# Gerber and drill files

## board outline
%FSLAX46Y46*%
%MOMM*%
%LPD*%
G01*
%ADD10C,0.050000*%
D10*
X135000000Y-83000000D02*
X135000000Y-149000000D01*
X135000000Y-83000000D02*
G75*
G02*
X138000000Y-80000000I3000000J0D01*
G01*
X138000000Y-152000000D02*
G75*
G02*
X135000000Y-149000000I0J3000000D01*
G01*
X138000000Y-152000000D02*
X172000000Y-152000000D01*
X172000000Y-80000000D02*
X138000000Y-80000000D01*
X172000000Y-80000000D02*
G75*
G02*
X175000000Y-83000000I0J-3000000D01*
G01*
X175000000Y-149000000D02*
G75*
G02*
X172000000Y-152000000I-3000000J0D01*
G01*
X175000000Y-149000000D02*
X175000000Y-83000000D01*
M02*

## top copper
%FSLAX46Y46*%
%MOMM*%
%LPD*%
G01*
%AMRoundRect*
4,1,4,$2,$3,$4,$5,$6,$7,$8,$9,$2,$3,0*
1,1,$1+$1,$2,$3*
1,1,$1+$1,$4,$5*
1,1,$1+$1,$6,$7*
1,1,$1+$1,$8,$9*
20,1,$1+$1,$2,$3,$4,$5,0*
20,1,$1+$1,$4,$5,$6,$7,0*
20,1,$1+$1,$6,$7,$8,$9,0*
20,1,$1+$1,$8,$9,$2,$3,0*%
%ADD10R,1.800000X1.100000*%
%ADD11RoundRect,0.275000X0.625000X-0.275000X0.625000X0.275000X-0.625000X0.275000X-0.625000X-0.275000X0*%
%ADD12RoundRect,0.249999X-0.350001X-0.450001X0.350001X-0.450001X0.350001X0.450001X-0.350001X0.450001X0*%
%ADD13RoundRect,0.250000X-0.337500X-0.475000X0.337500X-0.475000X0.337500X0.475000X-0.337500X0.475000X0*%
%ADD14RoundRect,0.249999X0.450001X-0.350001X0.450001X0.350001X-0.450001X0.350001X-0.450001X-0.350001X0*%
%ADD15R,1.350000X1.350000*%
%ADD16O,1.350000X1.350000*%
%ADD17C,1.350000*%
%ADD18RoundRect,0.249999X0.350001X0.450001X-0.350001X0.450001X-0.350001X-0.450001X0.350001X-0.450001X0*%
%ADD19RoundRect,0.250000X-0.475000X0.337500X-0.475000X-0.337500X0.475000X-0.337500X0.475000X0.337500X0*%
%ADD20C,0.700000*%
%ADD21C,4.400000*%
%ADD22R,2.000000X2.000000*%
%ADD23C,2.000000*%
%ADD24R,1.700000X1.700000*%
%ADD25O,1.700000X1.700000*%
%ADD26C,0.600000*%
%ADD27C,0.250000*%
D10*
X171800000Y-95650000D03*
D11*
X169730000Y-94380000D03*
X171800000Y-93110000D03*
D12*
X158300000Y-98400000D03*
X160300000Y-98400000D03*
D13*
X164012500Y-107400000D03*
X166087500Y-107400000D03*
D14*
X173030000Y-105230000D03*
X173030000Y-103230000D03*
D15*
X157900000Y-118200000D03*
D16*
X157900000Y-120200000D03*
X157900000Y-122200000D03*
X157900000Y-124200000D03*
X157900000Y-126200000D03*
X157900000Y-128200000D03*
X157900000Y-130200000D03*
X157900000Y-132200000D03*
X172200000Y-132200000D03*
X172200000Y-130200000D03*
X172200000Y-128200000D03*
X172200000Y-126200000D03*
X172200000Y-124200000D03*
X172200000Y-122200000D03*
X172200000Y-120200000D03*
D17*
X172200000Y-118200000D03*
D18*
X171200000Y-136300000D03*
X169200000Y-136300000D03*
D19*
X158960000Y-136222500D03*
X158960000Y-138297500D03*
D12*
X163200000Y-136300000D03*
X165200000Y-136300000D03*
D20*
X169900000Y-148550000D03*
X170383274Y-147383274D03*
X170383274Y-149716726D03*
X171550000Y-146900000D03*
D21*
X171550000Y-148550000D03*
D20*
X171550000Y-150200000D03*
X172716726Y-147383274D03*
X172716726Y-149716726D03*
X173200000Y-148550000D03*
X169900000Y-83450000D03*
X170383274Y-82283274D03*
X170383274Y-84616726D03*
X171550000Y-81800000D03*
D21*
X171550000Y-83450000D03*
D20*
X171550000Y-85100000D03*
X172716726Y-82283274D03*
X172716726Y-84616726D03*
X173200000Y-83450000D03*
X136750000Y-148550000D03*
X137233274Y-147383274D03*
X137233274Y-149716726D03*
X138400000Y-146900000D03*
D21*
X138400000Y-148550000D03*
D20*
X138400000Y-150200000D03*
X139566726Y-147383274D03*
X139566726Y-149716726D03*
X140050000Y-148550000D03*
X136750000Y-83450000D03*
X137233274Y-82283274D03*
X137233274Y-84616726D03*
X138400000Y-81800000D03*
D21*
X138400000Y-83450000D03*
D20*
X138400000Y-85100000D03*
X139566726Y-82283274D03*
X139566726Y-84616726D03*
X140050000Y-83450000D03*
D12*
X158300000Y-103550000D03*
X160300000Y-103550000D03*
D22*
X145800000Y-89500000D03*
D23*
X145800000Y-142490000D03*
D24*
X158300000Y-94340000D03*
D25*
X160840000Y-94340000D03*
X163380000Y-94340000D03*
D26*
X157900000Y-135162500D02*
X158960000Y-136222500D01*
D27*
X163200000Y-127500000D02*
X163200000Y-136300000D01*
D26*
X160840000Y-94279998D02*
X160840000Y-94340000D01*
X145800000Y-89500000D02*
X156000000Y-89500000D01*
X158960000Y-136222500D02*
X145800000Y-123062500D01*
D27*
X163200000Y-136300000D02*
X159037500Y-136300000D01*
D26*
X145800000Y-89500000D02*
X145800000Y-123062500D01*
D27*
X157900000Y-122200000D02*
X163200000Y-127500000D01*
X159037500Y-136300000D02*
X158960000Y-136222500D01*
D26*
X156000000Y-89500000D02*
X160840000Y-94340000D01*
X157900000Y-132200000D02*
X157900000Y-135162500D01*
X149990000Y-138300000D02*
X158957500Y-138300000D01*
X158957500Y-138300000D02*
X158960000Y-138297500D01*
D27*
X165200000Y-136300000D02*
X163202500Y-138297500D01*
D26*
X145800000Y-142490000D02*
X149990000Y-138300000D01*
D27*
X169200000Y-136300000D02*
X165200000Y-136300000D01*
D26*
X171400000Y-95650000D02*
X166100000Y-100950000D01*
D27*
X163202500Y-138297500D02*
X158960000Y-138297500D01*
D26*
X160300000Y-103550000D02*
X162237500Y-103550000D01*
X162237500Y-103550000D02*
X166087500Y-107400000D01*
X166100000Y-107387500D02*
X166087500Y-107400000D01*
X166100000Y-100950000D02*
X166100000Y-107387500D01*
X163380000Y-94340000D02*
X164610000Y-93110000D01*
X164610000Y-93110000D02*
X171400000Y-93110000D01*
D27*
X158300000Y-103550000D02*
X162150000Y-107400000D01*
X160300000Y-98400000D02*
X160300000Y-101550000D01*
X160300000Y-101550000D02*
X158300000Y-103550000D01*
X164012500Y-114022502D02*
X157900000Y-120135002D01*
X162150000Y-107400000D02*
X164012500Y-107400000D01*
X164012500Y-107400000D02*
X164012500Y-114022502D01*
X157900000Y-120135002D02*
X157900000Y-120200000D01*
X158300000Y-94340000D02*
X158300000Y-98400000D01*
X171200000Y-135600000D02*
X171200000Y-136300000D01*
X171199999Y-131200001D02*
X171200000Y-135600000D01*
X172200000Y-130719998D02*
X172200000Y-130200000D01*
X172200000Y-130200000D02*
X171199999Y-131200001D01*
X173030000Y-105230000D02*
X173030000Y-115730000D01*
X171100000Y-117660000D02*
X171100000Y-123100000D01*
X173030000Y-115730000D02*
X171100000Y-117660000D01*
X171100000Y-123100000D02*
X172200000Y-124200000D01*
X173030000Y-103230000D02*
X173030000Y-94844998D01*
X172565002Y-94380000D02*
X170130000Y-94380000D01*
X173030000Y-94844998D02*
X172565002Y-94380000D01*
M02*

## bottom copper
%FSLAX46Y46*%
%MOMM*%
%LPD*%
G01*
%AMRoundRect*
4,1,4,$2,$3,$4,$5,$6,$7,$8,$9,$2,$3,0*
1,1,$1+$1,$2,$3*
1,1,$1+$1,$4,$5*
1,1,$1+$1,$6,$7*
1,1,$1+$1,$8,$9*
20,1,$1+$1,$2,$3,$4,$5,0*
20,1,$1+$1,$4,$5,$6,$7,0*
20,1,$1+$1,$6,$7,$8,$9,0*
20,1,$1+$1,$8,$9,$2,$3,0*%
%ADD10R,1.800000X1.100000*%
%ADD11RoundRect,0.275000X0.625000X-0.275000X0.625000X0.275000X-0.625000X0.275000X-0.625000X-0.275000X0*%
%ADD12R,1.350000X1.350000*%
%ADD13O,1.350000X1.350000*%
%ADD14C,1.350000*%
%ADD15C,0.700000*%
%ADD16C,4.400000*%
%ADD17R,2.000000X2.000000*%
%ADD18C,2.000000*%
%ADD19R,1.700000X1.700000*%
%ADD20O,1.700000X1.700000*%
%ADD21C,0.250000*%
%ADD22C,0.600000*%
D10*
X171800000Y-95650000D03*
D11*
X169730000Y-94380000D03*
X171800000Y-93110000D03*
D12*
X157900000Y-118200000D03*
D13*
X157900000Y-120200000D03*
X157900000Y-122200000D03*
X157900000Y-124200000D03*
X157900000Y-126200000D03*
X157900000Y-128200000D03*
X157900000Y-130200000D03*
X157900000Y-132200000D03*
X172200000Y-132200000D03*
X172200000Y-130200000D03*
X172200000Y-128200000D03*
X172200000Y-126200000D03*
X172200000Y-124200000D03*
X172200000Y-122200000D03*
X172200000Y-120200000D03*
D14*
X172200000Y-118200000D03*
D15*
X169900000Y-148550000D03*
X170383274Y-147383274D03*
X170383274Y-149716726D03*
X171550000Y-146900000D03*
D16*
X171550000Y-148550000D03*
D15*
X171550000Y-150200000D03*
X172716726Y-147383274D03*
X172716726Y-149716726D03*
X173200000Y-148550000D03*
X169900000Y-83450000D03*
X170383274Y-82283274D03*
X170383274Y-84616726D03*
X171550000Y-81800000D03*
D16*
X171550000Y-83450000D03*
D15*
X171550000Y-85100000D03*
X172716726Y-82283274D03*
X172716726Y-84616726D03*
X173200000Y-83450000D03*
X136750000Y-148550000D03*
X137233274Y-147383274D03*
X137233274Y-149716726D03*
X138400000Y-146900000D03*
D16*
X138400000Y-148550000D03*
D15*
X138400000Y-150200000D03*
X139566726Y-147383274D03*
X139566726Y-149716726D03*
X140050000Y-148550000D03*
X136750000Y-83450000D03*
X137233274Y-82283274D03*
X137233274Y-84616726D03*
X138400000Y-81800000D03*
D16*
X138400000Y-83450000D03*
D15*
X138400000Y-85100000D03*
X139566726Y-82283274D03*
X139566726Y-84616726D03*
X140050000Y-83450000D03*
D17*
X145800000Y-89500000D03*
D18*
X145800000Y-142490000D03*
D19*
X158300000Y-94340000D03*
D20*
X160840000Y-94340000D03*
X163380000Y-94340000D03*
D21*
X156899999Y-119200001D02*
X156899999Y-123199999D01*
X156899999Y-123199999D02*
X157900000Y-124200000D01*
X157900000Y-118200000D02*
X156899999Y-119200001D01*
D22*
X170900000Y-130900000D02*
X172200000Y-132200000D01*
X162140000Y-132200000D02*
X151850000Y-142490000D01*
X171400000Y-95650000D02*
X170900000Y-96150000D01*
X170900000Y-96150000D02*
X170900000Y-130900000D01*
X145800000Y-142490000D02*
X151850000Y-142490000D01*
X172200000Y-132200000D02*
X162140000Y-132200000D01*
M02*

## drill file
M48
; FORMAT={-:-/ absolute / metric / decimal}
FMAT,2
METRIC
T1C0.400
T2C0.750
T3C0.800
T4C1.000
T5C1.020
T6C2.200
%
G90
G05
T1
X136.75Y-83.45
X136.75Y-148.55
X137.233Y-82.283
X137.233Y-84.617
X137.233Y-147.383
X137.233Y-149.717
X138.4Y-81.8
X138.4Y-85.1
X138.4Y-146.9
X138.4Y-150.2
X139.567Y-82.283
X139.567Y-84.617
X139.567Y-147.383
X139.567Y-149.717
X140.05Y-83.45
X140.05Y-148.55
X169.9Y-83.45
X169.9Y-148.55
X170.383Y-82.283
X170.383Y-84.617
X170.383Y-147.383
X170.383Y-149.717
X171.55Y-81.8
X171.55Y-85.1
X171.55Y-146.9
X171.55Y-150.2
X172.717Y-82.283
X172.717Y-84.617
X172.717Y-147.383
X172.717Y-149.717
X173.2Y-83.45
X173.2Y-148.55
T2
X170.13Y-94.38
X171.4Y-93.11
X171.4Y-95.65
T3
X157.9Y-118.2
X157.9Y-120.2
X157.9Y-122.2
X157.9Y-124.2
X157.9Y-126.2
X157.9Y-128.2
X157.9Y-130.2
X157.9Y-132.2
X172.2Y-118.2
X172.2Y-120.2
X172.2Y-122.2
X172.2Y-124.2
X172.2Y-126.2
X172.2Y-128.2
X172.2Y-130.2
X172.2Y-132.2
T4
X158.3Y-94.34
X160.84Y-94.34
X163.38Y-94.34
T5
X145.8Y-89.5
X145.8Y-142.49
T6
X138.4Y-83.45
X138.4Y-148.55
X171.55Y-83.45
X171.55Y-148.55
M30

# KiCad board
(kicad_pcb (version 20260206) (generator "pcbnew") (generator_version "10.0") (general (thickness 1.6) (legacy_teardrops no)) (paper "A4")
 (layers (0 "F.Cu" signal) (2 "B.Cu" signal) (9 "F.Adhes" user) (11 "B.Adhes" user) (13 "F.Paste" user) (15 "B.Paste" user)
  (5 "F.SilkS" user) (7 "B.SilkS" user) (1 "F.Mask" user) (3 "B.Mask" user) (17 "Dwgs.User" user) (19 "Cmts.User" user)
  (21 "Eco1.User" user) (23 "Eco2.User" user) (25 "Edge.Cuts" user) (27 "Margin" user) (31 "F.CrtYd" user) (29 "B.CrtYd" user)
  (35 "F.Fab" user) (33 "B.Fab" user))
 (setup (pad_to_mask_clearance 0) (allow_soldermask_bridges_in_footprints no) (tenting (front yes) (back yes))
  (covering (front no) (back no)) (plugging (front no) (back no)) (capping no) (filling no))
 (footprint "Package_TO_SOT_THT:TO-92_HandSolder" (layer "F.Cu") (at 171.4 95.65 90)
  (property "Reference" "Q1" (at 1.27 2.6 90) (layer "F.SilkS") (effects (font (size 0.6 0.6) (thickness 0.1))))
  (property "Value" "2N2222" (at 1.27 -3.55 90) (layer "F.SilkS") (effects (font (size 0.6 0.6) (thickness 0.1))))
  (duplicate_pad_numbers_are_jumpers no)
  (pad "1" thru_hole rect (at 0 0 90) (size 1.1 1.8) (drill 0.75 (offset 0 0.4)) (layers "*.Cu" "*.Mask") (remove_unused_layers no)
   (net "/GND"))
  (pad "2" thru_hole roundrect (at 1.27 -1.27 90) (size 1.1 1.8) (drill 0.75 (offset 0 -0.4)) (layers "*.Cu" "*.Mask")
   (remove_unused_layers no) (roundrect_rratio 0.25) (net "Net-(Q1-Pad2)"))
  (pad "3" thru_hole roundrect (at 2.54 0 90) (size 1.1 1.8) (drill 0.75 (offset 0 0.4)) (layers "*.Cu" "*.Mask") (remove_unused_layers no)
   (roundrect_rratio 0.25) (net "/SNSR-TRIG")))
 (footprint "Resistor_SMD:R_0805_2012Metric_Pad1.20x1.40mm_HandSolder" (layer "F.Cu") (at 159.3 98.4)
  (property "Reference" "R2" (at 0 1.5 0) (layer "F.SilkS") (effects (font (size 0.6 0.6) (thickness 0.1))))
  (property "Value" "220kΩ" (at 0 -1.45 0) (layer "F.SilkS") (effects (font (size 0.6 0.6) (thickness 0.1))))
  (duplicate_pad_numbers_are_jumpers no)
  (pad "1" smd roundrect (at -1 0) (size 1.2 1.4) (layers "F.Cu" "F.Mask" "F.Paste") (roundrect_rratio 0.2083325) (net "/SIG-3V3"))
  (pad "2" smd roundrect (at 1 0) (size 1.2 1.4) (layers "F.Cu" "F.Mask" "F.Paste") (roundrect_rratio 0.2083325) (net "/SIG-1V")))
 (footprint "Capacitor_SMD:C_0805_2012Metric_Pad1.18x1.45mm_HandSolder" (layer "F.Cu") (at 165.05 107.4)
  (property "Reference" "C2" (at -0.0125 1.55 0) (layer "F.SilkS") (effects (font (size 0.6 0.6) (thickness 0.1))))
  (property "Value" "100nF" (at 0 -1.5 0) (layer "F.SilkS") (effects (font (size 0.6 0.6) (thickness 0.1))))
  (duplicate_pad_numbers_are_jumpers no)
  (pad "1" smd roundrect (at -1.0375 0) (size 1.175 1.45) (layers "F.Cu" "F.Mask" "F.Paste") (roundrect_rratio 0.2127659574) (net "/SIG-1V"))
  (pad "2" smd roundrect (at 1.0375 0) (size 1.175 1.45) (layers "F.Cu" "F.Mask" "F.Paste") (roundrect_rratio 0.2127659574) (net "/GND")))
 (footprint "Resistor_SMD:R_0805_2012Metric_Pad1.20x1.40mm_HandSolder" (layer "F.Cu") (at 173.03 104.23 90)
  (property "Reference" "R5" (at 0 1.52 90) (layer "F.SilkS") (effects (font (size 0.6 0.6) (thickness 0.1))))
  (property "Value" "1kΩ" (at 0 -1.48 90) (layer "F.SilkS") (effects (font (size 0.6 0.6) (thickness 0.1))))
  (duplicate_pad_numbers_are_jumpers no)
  (pad "1" smd roundrect (at -1 0 90) (size 1.2 1.4) (layers "F.Cu" "F.Mask" "F.Paste") (roundrect_rratio 0.2083325) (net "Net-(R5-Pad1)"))
  (pad "2" smd roundrect (at 1 0 90) (size 1.2 1.4) (layers "F.Cu" "F.Mask" "F.Paste") (roundrect_rratio 0.2083325) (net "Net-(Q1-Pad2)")))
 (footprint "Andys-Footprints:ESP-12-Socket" (layer "F.Cu") (at 157.9 118.2)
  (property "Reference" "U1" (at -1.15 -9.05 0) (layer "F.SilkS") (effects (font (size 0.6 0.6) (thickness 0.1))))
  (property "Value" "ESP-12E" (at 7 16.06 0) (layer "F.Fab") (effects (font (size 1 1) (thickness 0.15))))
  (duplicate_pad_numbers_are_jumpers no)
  (pad "1" thru_hole rect (at 0 0) (size 1.35 1.35) (drill 0.8) (layers "*.Cu" "*.Mask") (remove_unused_layers no) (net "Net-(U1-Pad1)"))
  (pad "2" thru_hole oval (at 0 2) (size 1.35 1.35) (drill 0.8) (layers "*.Cu" "*.Mask") (remove_unused_layers no) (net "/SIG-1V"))
  (pad "3" thru_hole oval (at 0 4) (size 1.35 1.35) (drill 0.8) (layers "*.Cu" "*.Mask") (remove_unused_layers no) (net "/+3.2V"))
  (pad "4" thru_hole oval (at 0 6) (size 1.35 1.35) (drill 0.8) (layers "*.Cu" "*.Mask") (remove_unused_layers no) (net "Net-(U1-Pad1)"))
  (pad "5" thru_hole oval (at 0 8) (size 1.35 1.35) (drill 0.8) (layers "*.Cu" "*.Mask") (remove_unused_layers no))
  (pad "6" thru_hole oval (at 0 10) (size 1.35 1.35) (drill 0.8) (layers "*.Cu" "*.Mask") (remove_unused_layers no))
  (pad "7" thru_hole oval (at 0 12) (size 1.35 1.35) (drill 0.8) (layers "*.Cu" "*.Mask") (remove_unused_layers no))
  (pad "8" thru_hole oval (at 0 14) (size 1.35 1.35) (drill 0.8) (layers "*.Cu" "*.Mask") (remove_unused_layers no) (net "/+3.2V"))
  (pad "15" thru_hole oval (at 14.3 14) (size 1.35 1.35) (drill 0.8) (layers "*.Cu" "*.Mask") (remove_unused_layers no) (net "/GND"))
  (pad "16" thru_hole oval (at 14.3 12) (size 1.35 1.35) (drill 0.8) (layers "*.Cu" "*.Mask") (remove_unused_layers no) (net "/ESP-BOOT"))
  (pad "17" thru_hole oval (at 14.3 10) (size 1.35 1.35) (drill 0.8) (layers "*.Cu" "*.Mask") (remove_unused_layers no))
  (pad "18" thru_hole oval (at 14.3 8) (size 1.35 1.35) (drill 0.8) (layers "*.Cu" "*.Mask") (remove_unused_layers no))
  (pad "19" thru_hole oval (at 14.3 6) (size 1.35 1.35) (drill 0.8) (layers "*.Cu" "*.Mask") (remove_unused_layers no) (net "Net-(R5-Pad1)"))
  (pad "20" thru_hole oval (at 14.3 4) (size 1.35 1.35) (drill 0.8) (layers "*.Cu" "*.Mask") (remove_unused_layers no))
  (pad "21" thru_hole oval (at 14.3 2) (size 1.35 1.35) (drill 0.8) (layers "*.Cu" "*.Mask") (remove_unused_layers no))
  (pad "22" thru_hole circle (at 14.3 0) (size 1.35 1.35) (drill 0.8) (layers "*.Cu" "*.Mask") (remove_unused_layers no)))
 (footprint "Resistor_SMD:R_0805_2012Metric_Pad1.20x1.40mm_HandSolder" (layer "F.Cu") (at 170.2 136.3 180)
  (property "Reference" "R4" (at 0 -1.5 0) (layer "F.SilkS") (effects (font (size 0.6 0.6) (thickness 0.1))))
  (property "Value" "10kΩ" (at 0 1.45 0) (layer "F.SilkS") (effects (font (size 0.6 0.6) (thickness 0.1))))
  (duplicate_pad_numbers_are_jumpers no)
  (pad "1" smd roundrect (at -1 0 180) (size 1.2 1.4) (layers "F.Cu" "F.Mask" "F.Paste") (roundrect_rratio 0.2083325) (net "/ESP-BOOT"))
  (pad "2" smd roundrect (at 1 0 180) (size 1.2 1.4) (layers "F.Cu" "F.Mask" "F.Paste") (roundrect_rratio 0.2083325) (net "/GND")))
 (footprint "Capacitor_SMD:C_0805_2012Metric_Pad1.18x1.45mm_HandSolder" (layer "F.Cu") (at 158.96 137.26 -90)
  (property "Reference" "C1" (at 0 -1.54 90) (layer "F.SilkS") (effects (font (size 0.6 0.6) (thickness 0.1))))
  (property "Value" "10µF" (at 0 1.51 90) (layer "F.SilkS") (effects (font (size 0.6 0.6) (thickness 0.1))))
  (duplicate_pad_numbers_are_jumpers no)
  (pad "1" smd roundrect (at -1.0375 0 270) (size 1.175 1.45) (layers "F.Cu" "F.Mask" "F.Paste") (roundrect_rratio 0.2127659574)
   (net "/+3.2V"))
  (pad "2" smd roundrect (at 1.0375 0 270) (size 1.175 1.45) (layers "F.Cu" "F.Mask" "F.Paste") (roundrect_rratio 0.2127659574) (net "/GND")))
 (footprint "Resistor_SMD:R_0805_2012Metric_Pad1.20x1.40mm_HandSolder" (layer "F.Cu") (at 164.2 136.3)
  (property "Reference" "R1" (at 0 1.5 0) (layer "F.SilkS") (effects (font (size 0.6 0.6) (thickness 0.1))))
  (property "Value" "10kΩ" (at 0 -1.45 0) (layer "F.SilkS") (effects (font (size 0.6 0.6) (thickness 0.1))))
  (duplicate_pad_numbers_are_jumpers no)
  (pad "1" smd roundrect (at -1 0) (size 1.2 1.4) (layers "F.Cu" "F.Mask" "F.Paste") (roundrect_rratio 0.2083325) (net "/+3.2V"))
  (pad "2" smd roundrect (at 1 0) (size 1.2 1.4) (layers "F.Cu" "F.Mask" "F.Paste") (roundrect_rratio 0.2083325) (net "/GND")))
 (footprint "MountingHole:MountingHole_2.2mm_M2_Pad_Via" (layer "F.Cu") (at 171.55 148.55)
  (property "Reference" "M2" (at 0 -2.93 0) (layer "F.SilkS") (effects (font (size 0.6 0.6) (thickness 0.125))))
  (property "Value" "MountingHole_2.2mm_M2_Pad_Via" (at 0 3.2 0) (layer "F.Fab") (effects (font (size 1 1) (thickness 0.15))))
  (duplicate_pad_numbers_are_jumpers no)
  (pad "1" thru_hole circle (at -1.65 0) (size 0.7 0.7) (drill 0.4) (layers "*.Cu" "*.Mask") (remove_unused_layers no))
  (pad "1" thru_hole circle (at -1.166726 -1.166726) (size 0.7 0.7) (drill 0.4) (layers "*.Cu" "*.Mask") (remove_unused_layers no))
  (pad "1" thru_hole circle (at -1.166726 1.166726) (size 0.7 0.7) (drill 0.4) (layers "*.Cu" "*.Mask") (remove_unused_layers no))
  (pad "1" thru_hole circle (at 0 -1.65) (size 0.7 0.7) (drill 0.4) (layers "*.Cu" "*.Mask") (remove_unused_layers no))
  (pad "1" thru_hole circle (at 0 0) (size 4.4 4.4) (drill 2.2) (layers "*.Cu" "*.Mask") (remove_unused_layers no))
  (pad "1" thru_hole circle (at 0 1.65) (size 0.7 0.7) (drill 0.4) (layers "*.Cu" "*.Mask") (remove_unused_layers no))
  (pad "1" thru_hole circle (at 1.166726 -1.166726) (size 0.7 0.7) (drill 0.4) (layers "*.Cu" "*.Mask") (remove_unused_layers no))
  (pad "1" thru_hole circle (at 1.166726 1.166726) (size 0.7 0.7) (drill 0.4) (layers "*.Cu" "*.Mask") (remove_unused_layers no))
  (pad "1" thru_hole circle (at 1.65 0) (size 0.7 0.7) (drill 0.4) (layers "*.Cu" "*.Mask") (remove_unused_layers no)))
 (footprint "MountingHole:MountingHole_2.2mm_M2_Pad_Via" (layer "F.Cu") (at 171.55 83.45)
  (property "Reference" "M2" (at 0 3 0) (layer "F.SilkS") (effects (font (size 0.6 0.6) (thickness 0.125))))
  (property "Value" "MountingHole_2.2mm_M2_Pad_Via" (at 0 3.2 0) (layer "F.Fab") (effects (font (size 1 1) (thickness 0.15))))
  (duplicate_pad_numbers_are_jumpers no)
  (pad "1" thru_hole circle (at -1.65 0) (size 0.7 0.7) (drill 0.4) (layers "*.Cu" "*.Mask") (remove_unused_layers no))
  (pad "1" thru_hole circle (at -1.166726 -1.166726) (size 0.7 0.7) (drill 0.4) (layers "*.Cu" "*.Mask") (remove_unused_layers no))
  (pad "1" thru_hole circle (at -1.166726 1.166726) (size 0.7 0.7) (drill 0.4) (layers "*.Cu" "*.Mask") (remove_unused_layers no))
  (pad "1" thru_hole circle (at 0 -1.65) (size 0.7 0.7) (drill 0.4) (layers "*.Cu" "*.Mask") (remove_unused_layers no))
  (pad "1" thru_hole circle (at 0 0) (size 4.4 4.4) (drill 2.2) (layers "*.Cu" "*.Mask") (remove_unused_layers no))
  (pad "1" thru_hole circle (at 0 1.65) (size 0.7 0.7) (drill 0.4) (layers "*.Cu" "*.Mask") (remove_unused_layers no))
  (pad "1" thru_hole circle (at 1.166726 -1.166726) (size 0.7 0.7) (drill 0.4) (layers "*.Cu" "*.Mask") (remove_unused_layers no))
  (pad "1" thru_hole circle (at 1.166726 1.166726) (size 0.7 0.7) (drill 0.4) (layers "*.Cu" "*.Mask") (remove_unused_layers no))
  (pad "1" thru_hole circle (at 1.65 0) (size 0.7 0.7) (drill 0.4) (layers "*.Cu" "*.Mask") (remove_unused_layers no)))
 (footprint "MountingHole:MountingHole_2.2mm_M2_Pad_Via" (layer "F.Cu") (at 138.4 148.55)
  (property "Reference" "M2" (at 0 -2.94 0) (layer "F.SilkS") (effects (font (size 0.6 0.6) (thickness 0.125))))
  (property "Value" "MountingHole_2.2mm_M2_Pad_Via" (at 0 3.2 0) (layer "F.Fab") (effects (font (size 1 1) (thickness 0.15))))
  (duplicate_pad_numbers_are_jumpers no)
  (pad "1" thru_hole circle (at -1.65 0) (size 0.7 0.7) (drill 0.4) (layers "*.Cu" "*.Mask") (remove_unused_layers no))
  (pad "1" thru_hole circle (at -1.166726 -1.166726) (size 0.7 0.7) (drill 0.4) (layers "*.Cu" "*.Mask") (remove_unused_layers no))
  (pad "1" thru_hole circle (at -1.166726 1.166726) (size 0.7 0.7) (drill 0.4) (layers "*.Cu" "*.Mask") (remove_unused_layers no))
  (pad "1" thru_hole circle (at 0 -1.65) (size 0.7 0.7) (drill 0.4) (layers "*.Cu" "*.Mask") (remove_unused_layers no))
  (pad "1" thru_hole circle (at 0 0) (size 4.4 4.4) (drill 2.2) (layers "*.Cu" "*.Mask") (remove_unused_layers no))
  (pad "1" thru_hole circle (at 0 1.65) (size 0.7 0.7) (drill 0.4) (layers "*.Cu" "*.Mask") (remove_unused_layers no))
  (pad "1" thru_hole circle (at 1.166726 -1.166726) (size 0.7 0.7) (drill 0.4) (layers "*.Cu" "*.Mask") (remove_unused_layers no))
  (pad "1" thru_hole circle (at 1.166726 1.166726) (size 0.7 0.7) (drill 0.4) (layers "*.Cu" "*.Mask") (remove_unused_layers no))
  (pad "1" thru_hole circle (at 1.65 0) (size 0.7 0.7) (drill 0.4) (layers "*.Cu" "*.Mask") (remove_unused_layers no)))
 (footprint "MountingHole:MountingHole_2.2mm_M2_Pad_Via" (layer "F.Cu") (at 138.4 83.45)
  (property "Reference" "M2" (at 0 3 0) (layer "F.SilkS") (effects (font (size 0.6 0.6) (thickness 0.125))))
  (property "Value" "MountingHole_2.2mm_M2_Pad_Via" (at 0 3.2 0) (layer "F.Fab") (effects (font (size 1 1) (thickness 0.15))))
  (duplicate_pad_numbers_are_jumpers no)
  (pad "1" thru_hole circle (at -1.65 0) (size 0.7 0.7) (drill 0.4) (layers "*.Cu" "*.Mask") (remove_unused_layers no))
  (pad "1" thru_hole circle (at -1.166726 -1.166726) (size 0.7 0.7) (drill 0.4) (layers "*.Cu" "*.Mask") (remove_unused_layers no))
  (pad "1" thru_hole circle (at -1.166726 1.166726) (size 0.7 0.7) (drill 0.4) (layers "*.Cu" "*.Mask") (remove_unused_layers no))
  (pad "1" thru_hole circle (at 0 -1.65) (size 0.7 0.7) (drill 0.4) (layers "*.Cu" "*.Mask") (remove_unused_layers no))
  (pad "1" thru_hole circle (at 0 0) (size 4.4 4.4) (drill 2.2) (layers "*.Cu" "*.Mask") (remove_unused_layers no))
  (pad "1" thru_hole circle (at 0 1.65) (size 0.7 0.7) (drill 0.4) (layers "*.Cu" "*.Mask") (remove_unused_layers no))
  (pad "1" thru_hole circle (at 1.166726 -1.166726) (size 0.7 0.7) (drill 0.4) (layers "*.Cu" "*.Mask") (remove_unused_layers no))
  (pad "1" thru_hole circle (at 1.166726 1.166726) (size 0.7 0.7) (drill 0.4) (layers "*.Cu" "*.Mask") (remove_unused_layers no))
  (pad "1" thru_hole circle (at 1.65 0) (size 0.7 0.7) (drill 0.4) (layers "*.Cu" "*.Mask") (remove_unused_layers no)))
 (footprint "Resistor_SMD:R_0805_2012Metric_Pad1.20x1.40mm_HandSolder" (layer "F.Cu") (at 159.3 103.55)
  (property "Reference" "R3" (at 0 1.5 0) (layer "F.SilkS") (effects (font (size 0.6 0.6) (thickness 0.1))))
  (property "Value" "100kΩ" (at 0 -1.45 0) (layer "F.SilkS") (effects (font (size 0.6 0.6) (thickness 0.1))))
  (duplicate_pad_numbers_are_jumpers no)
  (pad "1" smd roundrect (at -1 0) (size 1.2 1.4) (layers "F.Cu" "F.Mask" "F.Paste") (roundrect_rratio 0.2083325) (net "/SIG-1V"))
  (pad "2" smd roundrect (at 1 0) (size 1.2 1.4) (layers "F.Cu" "F.Mask" "F.Paste") (roundrect_rratio 0.2083325) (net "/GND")))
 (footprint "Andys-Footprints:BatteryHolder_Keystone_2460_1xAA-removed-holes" (layer "F.Cu") (at 145.8 90 -90)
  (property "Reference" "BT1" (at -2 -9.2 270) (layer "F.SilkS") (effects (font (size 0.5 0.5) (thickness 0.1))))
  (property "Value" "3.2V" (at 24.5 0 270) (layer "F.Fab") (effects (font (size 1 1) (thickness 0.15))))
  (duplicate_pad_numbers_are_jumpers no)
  (pad "1" thru_hole rect (at -0.5 0 90) (size 2 2) (drill 1.02) (layers "*.Cu" "*.Mask") (remove_unused_layers no) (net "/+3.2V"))
  (pad "2" thru_hole circle (at 52.49 0 90) (size 2 2) (drill 1.02) (layers "*.Cu" "*.Mask") (remove_unused_layers no) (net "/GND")))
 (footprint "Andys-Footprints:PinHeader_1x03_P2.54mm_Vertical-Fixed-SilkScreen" (layer "F.Cu") (at 158.3 94.34 90)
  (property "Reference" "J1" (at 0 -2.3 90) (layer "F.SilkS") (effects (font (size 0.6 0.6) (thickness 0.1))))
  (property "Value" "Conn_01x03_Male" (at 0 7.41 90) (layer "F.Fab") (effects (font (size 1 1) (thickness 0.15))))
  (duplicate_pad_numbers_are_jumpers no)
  (pad "1" thru_hole rect (at 0 0 90) (size 1.7 1.7) (drill 1) (layers "*.Cu" "*.Mask") (remove_unused_layers no) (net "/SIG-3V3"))
  (pad "2" thru_hole oval (at 0 2.54 90) (size 1.7 1.7) (drill 1) (layers "*.Cu" "*.Mask") (remove_unused_layers no) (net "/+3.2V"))
  (pad "3" thru_hole oval (at 0 5.08 90) (size 1.7 1.7) (drill 1) (layers "*.Cu" "*.Mask") (remove_unused_layers no) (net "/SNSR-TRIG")))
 (gr_line (start 135 83) (end 135 149) (stroke (width 0.05) (type solid)) (layer "Edge.Cuts"))
 (gr_arc (start 135 83) (mid 135.87868 80.87868) (end 138 80) (stroke (width 0.05) (type solid)) (layer "Edge.Cuts"))
 (gr_arc (start 138 152) (mid 135.87868 151.12132) (end 135 149) (stroke (width 0.05) (type solid)) (layer "Edge.Cuts"))
 (gr_line (start 138 152) (end 172 152) (stroke (width 0.05) (type solid)) (layer "Edge.Cuts"))
 (gr_line (start 172 80) (end 138 80) (stroke (width 0.05) (type solid)) (layer "Edge.Cuts"))
 (gr_arc (start 172 80) (mid 174.12132 80.87868) (end 175 83) (stroke (width 0.05) (type solid)) (layer "Edge.Cuts"))
 (gr_arc (start 175 149) (mid 174.12132 151.12132) (end 172 152) (stroke (width 0.05) (type solid)) (layer "Edge.Cuts"))
 (gr_line (start 175 149) (end 175 83) (stroke (width 0.05) (type solid)) (layer "Edge.Cuts"))
 (segment (start 156.899999 119.200001) (end 156.899999 123.199999) (width 0.25) (layer "B.Cu") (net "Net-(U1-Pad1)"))
 (segment (start 156.899999 123.199999) (end 157.9 124.2) (width 0.25) (layer "B.Cu") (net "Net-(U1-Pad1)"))
 (segment (start 157.9 118.2) (end 156.899999 119.200001) (width 0.25) (layer "B.Cu") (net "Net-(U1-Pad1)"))
 (segment (start 157.9 135.1625) (end 158.96 136.2225) (width 0.6) (layer "F.Cu") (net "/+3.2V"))
 (segment (start 163.2 127.5) (end 163.2 136.3) (width 0.25) (layer "F.Cu") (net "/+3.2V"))
 (segment (start 160.84 94.279998) (end 160.84 94.34) (width 0.6) (layer "F.Cu") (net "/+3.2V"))
 (segment (start 145.8 89.5) (end 156 89.5) (width 0.6) (layer "F.Cu") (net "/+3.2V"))
 (segment (start 158.96 136.2225) (end 145.8 123.0625) (width 0.6) (layer "F.Cu") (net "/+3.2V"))
 (segment (start 163.2 136.3) (end 159.0375 136.3) (width 0.25) (layer "F.Cu") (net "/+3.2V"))
 (segment (start 145.8 89.5) (end 145.8 123.0625) (width 0.6) (layer "F.Cu") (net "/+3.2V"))
 (segment (start 157.9 122.2) (end 163.2 127.5) (width 0.25) (layer "F.Cu") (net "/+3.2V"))
 (segment (start 159.0375 136.3) (end 158.96 136.2225) (width 0.25) (layer "F.Cu") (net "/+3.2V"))
 (segment (start 156 89.5) (end 160.84 94.34) (width 0.6) (layer "F.Cu") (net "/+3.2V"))
 (segment (start 157.9 132.2) (end 157.9 135.1625) (width 0.6) (layer "F.Cu") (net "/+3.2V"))
 (segment (start 149.99 138.3) (end 158.9575 138.3) (width 0.6) (layer "F.Cu") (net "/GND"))
 (segment (start 158.9575 138.3) (end 158.96 138.2975) (width 0.6) (layer "F.Cu") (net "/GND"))
 (segment (start 165.2 136.3) (end 163.2025 138.2975) (width 0.25) (layer "F.Cu") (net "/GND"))
 (segment (start 145.8 142.49) (end 149.99 138.3) (width 0.6) (layer "F.Cu") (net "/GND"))
 (segment (start 169.2 136.3) (end 165.2 136.3) (width 0.25) (layer "F.Cu") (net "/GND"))
 (segment (start 171.4 95.65) (end 166.1 100.95) (width 0.6) (layer "F.Cu") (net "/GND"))
 (segment (start 163.2025 138.2975) (end 158.96 138.2975) (width 0.25) (layer "F.Cu") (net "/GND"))
 (segment (start 160.3 103.55) (end 162.2375 103.55) (width 0.6) (layer "F.Cu") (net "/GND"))
 (segment (start 162.2375 103.55) (end 166.0875 107.4) (width 0.6) (layer "F.Cu") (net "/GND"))
 (segment (start 166.1 107.3875) (end 166.0875 107.4) (width 0.6) (layer "F.Cu") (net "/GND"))
 (segment (start 166.1 100.95) (end 166.1 107.3875) (width 0.6) (layer "F.Cu") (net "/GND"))
 (segment (start 170.9 130.9) (end 172.2 132.2) (width 0.6) (layer "B.Cu") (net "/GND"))
 (segment (start 162.14 132.2) (end 151.85 142.49) (width 0.6) (layer "B.Cu") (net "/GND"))
 (segment (start 171.4 95.65) (end 170.9 96.15) (width 0.6) (layer "B.Cu") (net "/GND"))
 (segment (start 170.9 96.15) (end 170.9 130.9) (width 0.6) (layer "B.Cu") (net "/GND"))
 (segment (start 145.8 142.49) (end 151.85 142.49) (width 0.6) (layer "B.Cu") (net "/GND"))
 (segment (start 172.2 132.2) (end 162.14 132.2) (width 0.6) (layer "B.Cu") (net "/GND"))
 (segment (start 163.38 94.34) (end 164.61 93.11) (width 0.6) (layer "F.Cu") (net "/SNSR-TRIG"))
 (segment (start 164.61 93.11) (end 171.4 93.11) (width 0.6) (layer "F.Cu") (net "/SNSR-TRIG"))
 (segment (start 158.3 103.55) (end 162.15 107.4) (width 0.25) (layer "F.Cu") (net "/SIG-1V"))
 (segment (start 160.3 98.4) (end 160.3 101.55) (width 0.25) (layer "F.Cu") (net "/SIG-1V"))
 (segment (start 160.3 101.55) (end 158.3 103.55) (width 0.25) (layer "F.Cu") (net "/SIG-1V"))
 (segment (start 164.0125 114.022502) (end 157.9 120.135002) (width 0.25) (layer "F.Cu") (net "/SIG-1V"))
 (segment (start 162.15 107.4) (end 164.0125 107.4) (width 0.25) (layer "F.Cu") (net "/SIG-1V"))
 (segment (start 164.0125 107.4) (end 164.0125 114.022502) (width 0.25) (layer "F.Cu") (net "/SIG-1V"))
 (segment (start 157.9 120.135002) (end 157.9 120.2) (width 0.25) (layer "F.Cu") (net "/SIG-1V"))
 (segment (start 158.3 94.34) (end 158.3 98.4) (width 0.25) (layer "F.Cu") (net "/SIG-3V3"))
 (segment (start 171.2 135.6) (end 171.2 136.3) (width 0.25) (layer "F.Cu") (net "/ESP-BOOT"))
 (segment (start 171.199999 131.200001) (end 171.2 135.6) (width 0.25) (layer "F.Cu") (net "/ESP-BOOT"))
 (segment (start 172.2 130.719998) (end 172.2 130.2) (width 0.25) (layer "F.Cu") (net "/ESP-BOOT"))
 (segment (start 172.2 130.2) (end 171.199999 131.200001) (width 0.25) (layer "F.Cu") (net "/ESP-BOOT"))
 (segment (start 173.03 105.23) (end 173.03 115.73) (width 0.25) (layer "F.Cu") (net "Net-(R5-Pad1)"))
 (segment (start 171.1 117.66) (end 171.1 123.1) (width 0.25) (layer "F.Cu") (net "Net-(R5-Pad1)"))
 (segment (start 173.03 115.73) (end 171.1 117.66) (width 0.25) (layer "F.Cu") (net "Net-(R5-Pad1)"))
 (segment (start 171.1 123.1) (end 172.2 124.2) (width 0.25) (layer "F.Cu") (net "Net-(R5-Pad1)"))
 (segment (start 173.03 103.23) (end 173.03 94.844998) (width 0.25) (layer "F.Cu") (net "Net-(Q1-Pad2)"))
 (segment (start 172.565002 94.38) (end 170.13 94.38) (width 0.25) (layer "F.Cu") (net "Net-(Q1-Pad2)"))
 (segment (start 173.03 94.844998) (end 172.565002 94.38) (width 0.25) (layer "F.Cu") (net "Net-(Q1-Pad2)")))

